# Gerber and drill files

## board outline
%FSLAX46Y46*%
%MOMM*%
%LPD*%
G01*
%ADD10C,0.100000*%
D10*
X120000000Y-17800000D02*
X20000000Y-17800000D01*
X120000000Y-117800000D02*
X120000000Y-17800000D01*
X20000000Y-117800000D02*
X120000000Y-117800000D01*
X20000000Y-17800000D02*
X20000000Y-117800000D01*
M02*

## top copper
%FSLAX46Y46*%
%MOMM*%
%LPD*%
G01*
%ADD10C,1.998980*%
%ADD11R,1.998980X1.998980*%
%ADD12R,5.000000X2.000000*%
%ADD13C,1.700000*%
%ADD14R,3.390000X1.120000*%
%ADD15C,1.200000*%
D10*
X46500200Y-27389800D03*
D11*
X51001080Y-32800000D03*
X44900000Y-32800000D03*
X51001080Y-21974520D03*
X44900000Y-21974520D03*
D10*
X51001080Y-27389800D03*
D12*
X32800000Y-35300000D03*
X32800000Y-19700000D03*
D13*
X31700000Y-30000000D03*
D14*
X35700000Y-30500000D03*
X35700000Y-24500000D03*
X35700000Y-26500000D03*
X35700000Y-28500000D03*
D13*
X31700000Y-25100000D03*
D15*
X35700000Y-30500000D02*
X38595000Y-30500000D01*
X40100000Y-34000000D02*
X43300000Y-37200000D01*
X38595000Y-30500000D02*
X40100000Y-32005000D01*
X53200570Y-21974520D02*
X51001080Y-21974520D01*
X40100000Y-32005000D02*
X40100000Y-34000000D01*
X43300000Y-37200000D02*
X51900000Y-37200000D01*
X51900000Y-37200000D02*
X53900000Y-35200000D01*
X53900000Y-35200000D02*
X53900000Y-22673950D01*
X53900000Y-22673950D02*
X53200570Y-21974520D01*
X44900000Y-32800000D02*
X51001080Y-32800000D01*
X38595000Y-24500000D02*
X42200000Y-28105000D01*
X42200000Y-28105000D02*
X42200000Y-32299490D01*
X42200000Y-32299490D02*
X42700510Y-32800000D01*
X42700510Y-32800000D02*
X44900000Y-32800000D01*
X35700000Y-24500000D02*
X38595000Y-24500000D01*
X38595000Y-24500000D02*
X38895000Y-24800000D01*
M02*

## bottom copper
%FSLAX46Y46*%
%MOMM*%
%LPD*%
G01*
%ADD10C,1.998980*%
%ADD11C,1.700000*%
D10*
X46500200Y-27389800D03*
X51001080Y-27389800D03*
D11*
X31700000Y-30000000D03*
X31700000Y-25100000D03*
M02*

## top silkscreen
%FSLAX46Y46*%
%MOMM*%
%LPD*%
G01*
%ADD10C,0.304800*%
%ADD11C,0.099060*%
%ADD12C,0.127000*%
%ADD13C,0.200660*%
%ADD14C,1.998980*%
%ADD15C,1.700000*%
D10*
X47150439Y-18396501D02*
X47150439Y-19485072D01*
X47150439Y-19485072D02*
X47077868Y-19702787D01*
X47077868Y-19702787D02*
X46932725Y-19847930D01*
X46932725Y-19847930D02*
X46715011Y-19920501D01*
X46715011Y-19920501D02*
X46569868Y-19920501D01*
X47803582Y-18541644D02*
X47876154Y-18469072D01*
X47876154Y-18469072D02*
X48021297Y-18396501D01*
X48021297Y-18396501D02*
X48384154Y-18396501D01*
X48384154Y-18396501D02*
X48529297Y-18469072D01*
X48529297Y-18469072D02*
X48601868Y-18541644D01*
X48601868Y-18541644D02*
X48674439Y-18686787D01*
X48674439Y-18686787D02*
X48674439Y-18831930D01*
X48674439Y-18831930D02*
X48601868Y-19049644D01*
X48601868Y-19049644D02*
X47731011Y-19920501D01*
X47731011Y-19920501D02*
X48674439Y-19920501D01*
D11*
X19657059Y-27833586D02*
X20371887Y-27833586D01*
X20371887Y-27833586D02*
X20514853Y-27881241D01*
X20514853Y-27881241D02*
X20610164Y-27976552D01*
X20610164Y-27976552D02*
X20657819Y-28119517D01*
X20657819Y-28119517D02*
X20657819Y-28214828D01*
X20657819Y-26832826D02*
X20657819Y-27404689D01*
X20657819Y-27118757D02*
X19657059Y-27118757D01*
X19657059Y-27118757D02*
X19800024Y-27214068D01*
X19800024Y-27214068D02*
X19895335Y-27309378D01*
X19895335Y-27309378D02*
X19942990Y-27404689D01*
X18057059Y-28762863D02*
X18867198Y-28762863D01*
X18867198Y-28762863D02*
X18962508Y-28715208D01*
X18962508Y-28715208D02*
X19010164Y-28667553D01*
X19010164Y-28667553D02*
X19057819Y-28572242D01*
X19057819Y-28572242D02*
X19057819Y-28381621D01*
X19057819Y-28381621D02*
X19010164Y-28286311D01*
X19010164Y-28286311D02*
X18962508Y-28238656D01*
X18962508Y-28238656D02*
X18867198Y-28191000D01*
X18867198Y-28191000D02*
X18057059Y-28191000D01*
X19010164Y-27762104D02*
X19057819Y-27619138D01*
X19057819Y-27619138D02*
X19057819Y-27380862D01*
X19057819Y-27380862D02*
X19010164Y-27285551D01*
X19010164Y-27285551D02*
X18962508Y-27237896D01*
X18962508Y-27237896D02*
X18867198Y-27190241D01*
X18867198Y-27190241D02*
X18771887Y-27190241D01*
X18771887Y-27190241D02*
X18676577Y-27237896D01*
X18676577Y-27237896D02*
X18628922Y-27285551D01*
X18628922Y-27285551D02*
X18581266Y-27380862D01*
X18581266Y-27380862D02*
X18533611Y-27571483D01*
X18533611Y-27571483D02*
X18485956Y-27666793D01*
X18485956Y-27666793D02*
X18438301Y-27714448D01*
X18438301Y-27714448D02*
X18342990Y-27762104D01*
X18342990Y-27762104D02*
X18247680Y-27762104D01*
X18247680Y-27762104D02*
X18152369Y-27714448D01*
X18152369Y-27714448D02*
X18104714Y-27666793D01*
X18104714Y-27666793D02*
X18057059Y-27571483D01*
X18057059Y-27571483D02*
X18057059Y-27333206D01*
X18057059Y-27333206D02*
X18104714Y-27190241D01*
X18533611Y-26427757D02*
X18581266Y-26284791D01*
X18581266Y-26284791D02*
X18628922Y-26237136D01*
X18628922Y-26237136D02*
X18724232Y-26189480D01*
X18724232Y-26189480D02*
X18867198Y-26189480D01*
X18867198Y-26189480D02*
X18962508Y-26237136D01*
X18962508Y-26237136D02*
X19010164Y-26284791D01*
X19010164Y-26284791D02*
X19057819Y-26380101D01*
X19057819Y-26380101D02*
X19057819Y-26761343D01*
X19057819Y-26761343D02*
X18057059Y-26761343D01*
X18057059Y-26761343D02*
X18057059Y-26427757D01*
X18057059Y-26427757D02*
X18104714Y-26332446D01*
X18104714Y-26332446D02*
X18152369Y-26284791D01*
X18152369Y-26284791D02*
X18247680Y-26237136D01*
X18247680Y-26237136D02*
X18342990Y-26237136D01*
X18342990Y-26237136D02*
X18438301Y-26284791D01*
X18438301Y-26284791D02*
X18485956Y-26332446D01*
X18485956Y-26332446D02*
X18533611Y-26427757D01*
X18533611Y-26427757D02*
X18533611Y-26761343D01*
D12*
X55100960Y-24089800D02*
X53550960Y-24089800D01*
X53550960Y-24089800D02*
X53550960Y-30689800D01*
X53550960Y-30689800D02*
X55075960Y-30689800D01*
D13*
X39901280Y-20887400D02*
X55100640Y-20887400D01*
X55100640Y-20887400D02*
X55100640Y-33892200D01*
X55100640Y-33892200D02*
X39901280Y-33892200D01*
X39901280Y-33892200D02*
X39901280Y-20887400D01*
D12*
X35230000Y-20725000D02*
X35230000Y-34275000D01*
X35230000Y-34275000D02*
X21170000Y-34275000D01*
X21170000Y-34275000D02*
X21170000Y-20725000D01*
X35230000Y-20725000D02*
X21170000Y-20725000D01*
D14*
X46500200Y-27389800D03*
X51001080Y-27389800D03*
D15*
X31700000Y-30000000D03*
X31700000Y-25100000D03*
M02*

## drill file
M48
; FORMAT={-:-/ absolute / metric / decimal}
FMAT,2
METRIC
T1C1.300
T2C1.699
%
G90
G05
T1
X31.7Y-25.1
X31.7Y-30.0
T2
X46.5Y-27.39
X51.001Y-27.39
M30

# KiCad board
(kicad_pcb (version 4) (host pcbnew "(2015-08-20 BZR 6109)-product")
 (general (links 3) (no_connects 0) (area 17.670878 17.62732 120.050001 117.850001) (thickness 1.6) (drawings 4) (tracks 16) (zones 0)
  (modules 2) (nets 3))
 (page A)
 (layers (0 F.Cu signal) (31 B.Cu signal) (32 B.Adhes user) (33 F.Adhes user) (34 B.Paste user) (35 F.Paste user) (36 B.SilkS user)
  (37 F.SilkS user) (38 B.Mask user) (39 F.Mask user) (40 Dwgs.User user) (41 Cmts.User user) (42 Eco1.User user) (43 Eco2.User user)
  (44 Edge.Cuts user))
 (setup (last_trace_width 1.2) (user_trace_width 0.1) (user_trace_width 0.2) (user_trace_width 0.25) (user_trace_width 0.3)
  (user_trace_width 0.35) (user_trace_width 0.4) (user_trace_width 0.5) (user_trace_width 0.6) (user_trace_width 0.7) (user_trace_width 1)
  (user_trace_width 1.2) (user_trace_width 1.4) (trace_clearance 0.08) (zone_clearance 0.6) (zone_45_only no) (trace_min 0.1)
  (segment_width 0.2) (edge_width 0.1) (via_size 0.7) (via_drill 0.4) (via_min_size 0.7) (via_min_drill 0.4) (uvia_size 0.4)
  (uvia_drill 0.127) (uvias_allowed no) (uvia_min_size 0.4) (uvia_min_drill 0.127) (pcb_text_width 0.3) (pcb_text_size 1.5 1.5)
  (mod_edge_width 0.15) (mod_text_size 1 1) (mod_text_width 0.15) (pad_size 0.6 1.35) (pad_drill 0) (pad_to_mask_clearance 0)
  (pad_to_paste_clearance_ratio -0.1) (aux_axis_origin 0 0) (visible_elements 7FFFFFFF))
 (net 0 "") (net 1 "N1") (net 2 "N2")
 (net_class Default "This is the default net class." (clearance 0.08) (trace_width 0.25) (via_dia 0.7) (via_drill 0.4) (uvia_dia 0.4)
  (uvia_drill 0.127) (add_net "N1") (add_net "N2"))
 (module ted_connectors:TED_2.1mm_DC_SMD (layer F.Cu) (at 47.50096 27.3898)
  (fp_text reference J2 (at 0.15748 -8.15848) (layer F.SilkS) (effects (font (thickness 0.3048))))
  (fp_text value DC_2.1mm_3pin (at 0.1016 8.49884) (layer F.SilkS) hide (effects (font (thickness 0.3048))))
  (fp_line (start 7.6 -3.3) (end 6.05 -3.3) (layer F.SilkS) (width 0.127))
  (fp_line (start 6.05 -3.3) (end 6.05 3.3) (layer F.SilkS) (width 0.127))
  (fp_line (start 6.05 3.3) (end 7.575 3.3) (layer F.SilkS) (width 0.127))
  (fp_line (start -7.59968 -6.5024) (end 7.59968 -6.5024) (layer F.SilkS) (width 0.20066))
  (fp_line (start 7.59968 -6.5024) (end 7.59968 6.5024) (layer F.SilkS) (width 0.20066))
  (fp_line (start 7.59968 6.5024) (end -7.59968 6.5024) (layer F.SilkS) (width 0.20066))
  (fp_line (start -7.59968 6.5024) (end -7.59968 -6.5024) (layer F.SilkS) (width 0.20066))
  (pad "" np_thru_hole circle (at -1.00076 0) (size 1.99898 1.99898) (drill 1.69926) (layers *.Cu *.Mask F.SilkS))
  (pad 1 smd rect (at 3.50012 5.4102) (size 1.99898 1.99898) (layers F.Cu F.Paste F.Mask) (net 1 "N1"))
  (pad 1 smd rect (at -2.60096 5.4102) (size 1.99898 1.99898) (layers F.Cu F.Paste F.Mask) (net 1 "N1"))
  (pad 2 smd rect (at 3.50012 -5.41528) (size 1.99898 1.99898) (layers F.Cu F.Paste F.Mask) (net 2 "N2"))
  (pad 3 smd rect (at -2.60096 -5.41528) (size 1.99898 1.99898) (layers F.Cu F.Paste F.Mask))
  (pad "" np_thru_hole circle (at 3.50012 0) (size 1.99898 1.99898) (drill 1.69926) (layers *.Cu *.Mask F.SilkS)))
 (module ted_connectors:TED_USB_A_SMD (layer F.Cu) (at 28.2 27.5 270)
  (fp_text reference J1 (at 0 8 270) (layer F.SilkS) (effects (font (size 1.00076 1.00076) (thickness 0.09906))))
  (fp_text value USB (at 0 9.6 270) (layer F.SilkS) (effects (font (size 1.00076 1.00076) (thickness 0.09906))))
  (fp_line (start -6.775 -7.03) (end 6.775 -7.03) (layer F.SilkS) (width 0.127))
  (fp_line (start 6.775 -7.03) (end 6.775 7.03) (layer F.SilkS) (width 0.127))
  (fp_line (start 6.775 7.03) (end -6.775 7.03) (layer F.SilkS) (width 0.127))
  (fp_line (start -6.775 -7.03) (end -6.775 7.03) (layer F.SilkS) (width 0.127))
  (pad GP smd rect (at 7.8 -4.6 270) (size 2 5) (layers F.Cu F.Paste F.Mask))
  (pad GP smd rect (at -7.8 -4.6 270) (size 2 5) (layers F.Cu F.Paste F.Mask))
  (pad "" np_thru_hole circle (at 2.5 -3.5 270) (size 1.7 1.7) (drill 1.3) (layers *.Cu *.Mask F.SilkS))
  (pad 4 smd rect (at 3 -7.5 270) (size 1.12 3.39) (layers F.Cu F.Paste F.Mask) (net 2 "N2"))
  (pad 1 smd rect (at -3 -7.5 270) (size 1.12 3.39) (layers F.Cu F.Paste F.Mask) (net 1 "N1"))
  (pad 2 smd rect (at -1 -7.5 270) (size 1.12 3.39) (layers F.Cu F.Paste F.Mask))
  (pad 3 smd rect (at 1 -7.5 270) (size 1.12 3.39) (layers F.Cu F.Paste F.Mask))
  (pad "" np_thru_hole circle (at -2.4 -3.5 270) (size 1.7 1.7) (drill 1.3) (layers *.Cu *.Mask F.SilkS)))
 (gr_line (start 120 17.8) (end 20 17.8) (angle 90) (layer Edge.Cuts) (width 0.1))
 (gr_line (start 120 117.8) (end 120 17.8) (angle 90) (layer Edge.Cuts) (width 0.1))
 (gr_line (start 20 117.8) (end 120 117.8) (angle 90) (layer Edge.Cuts) (width 0.1))
 (gr_line (start 20 17.8) (end 20 117.8) (angle 90) (layer Edge.Cuts) (width 0.1))
 (segment (start 35.7 30.5) (end 38.595 30.5) (width 1.2) (layer F.Cu) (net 2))
 (segment (start 40.1 34) (end 43.3 37.2) (width 1.2) (layer F.Cu) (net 2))
 (segment (start 38.595 30.5) (end 40.1 32.005) (width 1.2) (layer F.Cu) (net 2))
 (segment (start 53.20057 21.97452) (end 51.00108 21.97452) (width 1.2) (layer F.Cu) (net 2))
 (segment (start 40.1 32.005) (end 40.1 34) (width 1.2) (layer F.Cu) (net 2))
 (segment (start 43.3 37.2) (end 51.9 37.2) (width 1.2) (layer F.Cu) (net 2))
 (segment (start 51.9 37.2) (end 53.9 35.2) (width 1.2) (layer F.Cu) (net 2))
 (segment (start 53.9 35.2) (end 53.9 22.67395) (width 1.2) (layer F.Cu) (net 2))
 (segment (start 53.9 22.67395) (end 53.20057 21.97452) (width 1.2) (layer F.Cu) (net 2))
 (segment (start 44.9 32.8) (end 51.00108 32.8) (width 1.2) (layer F.Cu) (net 1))
 (segment (start 38.595 24.5) (end 42.2 28.105) (width 1.2) (layer F.Cu) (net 1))
 (segment (start 42.2 28.105) (end 42.2 32.29949) (width 1.2) (layer F.Cu) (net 1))
 (segment (start 42.2 32.29949) (end 42.70051 32.8) (width 1.2) (layer F.Cu) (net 1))
 (segment (start 42.70051 32.8) (end 44.9 32.8) (width 1.2) (layer F.Cu) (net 1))
 (segment (start 35.7 24.5) (end 38.595 24.5) (width 1.2) (layer F.Cu) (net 1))
 (segment (start 38.595 24.5) (end 38.895 24.8) (width 1.2) (layer F.Cu) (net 1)))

